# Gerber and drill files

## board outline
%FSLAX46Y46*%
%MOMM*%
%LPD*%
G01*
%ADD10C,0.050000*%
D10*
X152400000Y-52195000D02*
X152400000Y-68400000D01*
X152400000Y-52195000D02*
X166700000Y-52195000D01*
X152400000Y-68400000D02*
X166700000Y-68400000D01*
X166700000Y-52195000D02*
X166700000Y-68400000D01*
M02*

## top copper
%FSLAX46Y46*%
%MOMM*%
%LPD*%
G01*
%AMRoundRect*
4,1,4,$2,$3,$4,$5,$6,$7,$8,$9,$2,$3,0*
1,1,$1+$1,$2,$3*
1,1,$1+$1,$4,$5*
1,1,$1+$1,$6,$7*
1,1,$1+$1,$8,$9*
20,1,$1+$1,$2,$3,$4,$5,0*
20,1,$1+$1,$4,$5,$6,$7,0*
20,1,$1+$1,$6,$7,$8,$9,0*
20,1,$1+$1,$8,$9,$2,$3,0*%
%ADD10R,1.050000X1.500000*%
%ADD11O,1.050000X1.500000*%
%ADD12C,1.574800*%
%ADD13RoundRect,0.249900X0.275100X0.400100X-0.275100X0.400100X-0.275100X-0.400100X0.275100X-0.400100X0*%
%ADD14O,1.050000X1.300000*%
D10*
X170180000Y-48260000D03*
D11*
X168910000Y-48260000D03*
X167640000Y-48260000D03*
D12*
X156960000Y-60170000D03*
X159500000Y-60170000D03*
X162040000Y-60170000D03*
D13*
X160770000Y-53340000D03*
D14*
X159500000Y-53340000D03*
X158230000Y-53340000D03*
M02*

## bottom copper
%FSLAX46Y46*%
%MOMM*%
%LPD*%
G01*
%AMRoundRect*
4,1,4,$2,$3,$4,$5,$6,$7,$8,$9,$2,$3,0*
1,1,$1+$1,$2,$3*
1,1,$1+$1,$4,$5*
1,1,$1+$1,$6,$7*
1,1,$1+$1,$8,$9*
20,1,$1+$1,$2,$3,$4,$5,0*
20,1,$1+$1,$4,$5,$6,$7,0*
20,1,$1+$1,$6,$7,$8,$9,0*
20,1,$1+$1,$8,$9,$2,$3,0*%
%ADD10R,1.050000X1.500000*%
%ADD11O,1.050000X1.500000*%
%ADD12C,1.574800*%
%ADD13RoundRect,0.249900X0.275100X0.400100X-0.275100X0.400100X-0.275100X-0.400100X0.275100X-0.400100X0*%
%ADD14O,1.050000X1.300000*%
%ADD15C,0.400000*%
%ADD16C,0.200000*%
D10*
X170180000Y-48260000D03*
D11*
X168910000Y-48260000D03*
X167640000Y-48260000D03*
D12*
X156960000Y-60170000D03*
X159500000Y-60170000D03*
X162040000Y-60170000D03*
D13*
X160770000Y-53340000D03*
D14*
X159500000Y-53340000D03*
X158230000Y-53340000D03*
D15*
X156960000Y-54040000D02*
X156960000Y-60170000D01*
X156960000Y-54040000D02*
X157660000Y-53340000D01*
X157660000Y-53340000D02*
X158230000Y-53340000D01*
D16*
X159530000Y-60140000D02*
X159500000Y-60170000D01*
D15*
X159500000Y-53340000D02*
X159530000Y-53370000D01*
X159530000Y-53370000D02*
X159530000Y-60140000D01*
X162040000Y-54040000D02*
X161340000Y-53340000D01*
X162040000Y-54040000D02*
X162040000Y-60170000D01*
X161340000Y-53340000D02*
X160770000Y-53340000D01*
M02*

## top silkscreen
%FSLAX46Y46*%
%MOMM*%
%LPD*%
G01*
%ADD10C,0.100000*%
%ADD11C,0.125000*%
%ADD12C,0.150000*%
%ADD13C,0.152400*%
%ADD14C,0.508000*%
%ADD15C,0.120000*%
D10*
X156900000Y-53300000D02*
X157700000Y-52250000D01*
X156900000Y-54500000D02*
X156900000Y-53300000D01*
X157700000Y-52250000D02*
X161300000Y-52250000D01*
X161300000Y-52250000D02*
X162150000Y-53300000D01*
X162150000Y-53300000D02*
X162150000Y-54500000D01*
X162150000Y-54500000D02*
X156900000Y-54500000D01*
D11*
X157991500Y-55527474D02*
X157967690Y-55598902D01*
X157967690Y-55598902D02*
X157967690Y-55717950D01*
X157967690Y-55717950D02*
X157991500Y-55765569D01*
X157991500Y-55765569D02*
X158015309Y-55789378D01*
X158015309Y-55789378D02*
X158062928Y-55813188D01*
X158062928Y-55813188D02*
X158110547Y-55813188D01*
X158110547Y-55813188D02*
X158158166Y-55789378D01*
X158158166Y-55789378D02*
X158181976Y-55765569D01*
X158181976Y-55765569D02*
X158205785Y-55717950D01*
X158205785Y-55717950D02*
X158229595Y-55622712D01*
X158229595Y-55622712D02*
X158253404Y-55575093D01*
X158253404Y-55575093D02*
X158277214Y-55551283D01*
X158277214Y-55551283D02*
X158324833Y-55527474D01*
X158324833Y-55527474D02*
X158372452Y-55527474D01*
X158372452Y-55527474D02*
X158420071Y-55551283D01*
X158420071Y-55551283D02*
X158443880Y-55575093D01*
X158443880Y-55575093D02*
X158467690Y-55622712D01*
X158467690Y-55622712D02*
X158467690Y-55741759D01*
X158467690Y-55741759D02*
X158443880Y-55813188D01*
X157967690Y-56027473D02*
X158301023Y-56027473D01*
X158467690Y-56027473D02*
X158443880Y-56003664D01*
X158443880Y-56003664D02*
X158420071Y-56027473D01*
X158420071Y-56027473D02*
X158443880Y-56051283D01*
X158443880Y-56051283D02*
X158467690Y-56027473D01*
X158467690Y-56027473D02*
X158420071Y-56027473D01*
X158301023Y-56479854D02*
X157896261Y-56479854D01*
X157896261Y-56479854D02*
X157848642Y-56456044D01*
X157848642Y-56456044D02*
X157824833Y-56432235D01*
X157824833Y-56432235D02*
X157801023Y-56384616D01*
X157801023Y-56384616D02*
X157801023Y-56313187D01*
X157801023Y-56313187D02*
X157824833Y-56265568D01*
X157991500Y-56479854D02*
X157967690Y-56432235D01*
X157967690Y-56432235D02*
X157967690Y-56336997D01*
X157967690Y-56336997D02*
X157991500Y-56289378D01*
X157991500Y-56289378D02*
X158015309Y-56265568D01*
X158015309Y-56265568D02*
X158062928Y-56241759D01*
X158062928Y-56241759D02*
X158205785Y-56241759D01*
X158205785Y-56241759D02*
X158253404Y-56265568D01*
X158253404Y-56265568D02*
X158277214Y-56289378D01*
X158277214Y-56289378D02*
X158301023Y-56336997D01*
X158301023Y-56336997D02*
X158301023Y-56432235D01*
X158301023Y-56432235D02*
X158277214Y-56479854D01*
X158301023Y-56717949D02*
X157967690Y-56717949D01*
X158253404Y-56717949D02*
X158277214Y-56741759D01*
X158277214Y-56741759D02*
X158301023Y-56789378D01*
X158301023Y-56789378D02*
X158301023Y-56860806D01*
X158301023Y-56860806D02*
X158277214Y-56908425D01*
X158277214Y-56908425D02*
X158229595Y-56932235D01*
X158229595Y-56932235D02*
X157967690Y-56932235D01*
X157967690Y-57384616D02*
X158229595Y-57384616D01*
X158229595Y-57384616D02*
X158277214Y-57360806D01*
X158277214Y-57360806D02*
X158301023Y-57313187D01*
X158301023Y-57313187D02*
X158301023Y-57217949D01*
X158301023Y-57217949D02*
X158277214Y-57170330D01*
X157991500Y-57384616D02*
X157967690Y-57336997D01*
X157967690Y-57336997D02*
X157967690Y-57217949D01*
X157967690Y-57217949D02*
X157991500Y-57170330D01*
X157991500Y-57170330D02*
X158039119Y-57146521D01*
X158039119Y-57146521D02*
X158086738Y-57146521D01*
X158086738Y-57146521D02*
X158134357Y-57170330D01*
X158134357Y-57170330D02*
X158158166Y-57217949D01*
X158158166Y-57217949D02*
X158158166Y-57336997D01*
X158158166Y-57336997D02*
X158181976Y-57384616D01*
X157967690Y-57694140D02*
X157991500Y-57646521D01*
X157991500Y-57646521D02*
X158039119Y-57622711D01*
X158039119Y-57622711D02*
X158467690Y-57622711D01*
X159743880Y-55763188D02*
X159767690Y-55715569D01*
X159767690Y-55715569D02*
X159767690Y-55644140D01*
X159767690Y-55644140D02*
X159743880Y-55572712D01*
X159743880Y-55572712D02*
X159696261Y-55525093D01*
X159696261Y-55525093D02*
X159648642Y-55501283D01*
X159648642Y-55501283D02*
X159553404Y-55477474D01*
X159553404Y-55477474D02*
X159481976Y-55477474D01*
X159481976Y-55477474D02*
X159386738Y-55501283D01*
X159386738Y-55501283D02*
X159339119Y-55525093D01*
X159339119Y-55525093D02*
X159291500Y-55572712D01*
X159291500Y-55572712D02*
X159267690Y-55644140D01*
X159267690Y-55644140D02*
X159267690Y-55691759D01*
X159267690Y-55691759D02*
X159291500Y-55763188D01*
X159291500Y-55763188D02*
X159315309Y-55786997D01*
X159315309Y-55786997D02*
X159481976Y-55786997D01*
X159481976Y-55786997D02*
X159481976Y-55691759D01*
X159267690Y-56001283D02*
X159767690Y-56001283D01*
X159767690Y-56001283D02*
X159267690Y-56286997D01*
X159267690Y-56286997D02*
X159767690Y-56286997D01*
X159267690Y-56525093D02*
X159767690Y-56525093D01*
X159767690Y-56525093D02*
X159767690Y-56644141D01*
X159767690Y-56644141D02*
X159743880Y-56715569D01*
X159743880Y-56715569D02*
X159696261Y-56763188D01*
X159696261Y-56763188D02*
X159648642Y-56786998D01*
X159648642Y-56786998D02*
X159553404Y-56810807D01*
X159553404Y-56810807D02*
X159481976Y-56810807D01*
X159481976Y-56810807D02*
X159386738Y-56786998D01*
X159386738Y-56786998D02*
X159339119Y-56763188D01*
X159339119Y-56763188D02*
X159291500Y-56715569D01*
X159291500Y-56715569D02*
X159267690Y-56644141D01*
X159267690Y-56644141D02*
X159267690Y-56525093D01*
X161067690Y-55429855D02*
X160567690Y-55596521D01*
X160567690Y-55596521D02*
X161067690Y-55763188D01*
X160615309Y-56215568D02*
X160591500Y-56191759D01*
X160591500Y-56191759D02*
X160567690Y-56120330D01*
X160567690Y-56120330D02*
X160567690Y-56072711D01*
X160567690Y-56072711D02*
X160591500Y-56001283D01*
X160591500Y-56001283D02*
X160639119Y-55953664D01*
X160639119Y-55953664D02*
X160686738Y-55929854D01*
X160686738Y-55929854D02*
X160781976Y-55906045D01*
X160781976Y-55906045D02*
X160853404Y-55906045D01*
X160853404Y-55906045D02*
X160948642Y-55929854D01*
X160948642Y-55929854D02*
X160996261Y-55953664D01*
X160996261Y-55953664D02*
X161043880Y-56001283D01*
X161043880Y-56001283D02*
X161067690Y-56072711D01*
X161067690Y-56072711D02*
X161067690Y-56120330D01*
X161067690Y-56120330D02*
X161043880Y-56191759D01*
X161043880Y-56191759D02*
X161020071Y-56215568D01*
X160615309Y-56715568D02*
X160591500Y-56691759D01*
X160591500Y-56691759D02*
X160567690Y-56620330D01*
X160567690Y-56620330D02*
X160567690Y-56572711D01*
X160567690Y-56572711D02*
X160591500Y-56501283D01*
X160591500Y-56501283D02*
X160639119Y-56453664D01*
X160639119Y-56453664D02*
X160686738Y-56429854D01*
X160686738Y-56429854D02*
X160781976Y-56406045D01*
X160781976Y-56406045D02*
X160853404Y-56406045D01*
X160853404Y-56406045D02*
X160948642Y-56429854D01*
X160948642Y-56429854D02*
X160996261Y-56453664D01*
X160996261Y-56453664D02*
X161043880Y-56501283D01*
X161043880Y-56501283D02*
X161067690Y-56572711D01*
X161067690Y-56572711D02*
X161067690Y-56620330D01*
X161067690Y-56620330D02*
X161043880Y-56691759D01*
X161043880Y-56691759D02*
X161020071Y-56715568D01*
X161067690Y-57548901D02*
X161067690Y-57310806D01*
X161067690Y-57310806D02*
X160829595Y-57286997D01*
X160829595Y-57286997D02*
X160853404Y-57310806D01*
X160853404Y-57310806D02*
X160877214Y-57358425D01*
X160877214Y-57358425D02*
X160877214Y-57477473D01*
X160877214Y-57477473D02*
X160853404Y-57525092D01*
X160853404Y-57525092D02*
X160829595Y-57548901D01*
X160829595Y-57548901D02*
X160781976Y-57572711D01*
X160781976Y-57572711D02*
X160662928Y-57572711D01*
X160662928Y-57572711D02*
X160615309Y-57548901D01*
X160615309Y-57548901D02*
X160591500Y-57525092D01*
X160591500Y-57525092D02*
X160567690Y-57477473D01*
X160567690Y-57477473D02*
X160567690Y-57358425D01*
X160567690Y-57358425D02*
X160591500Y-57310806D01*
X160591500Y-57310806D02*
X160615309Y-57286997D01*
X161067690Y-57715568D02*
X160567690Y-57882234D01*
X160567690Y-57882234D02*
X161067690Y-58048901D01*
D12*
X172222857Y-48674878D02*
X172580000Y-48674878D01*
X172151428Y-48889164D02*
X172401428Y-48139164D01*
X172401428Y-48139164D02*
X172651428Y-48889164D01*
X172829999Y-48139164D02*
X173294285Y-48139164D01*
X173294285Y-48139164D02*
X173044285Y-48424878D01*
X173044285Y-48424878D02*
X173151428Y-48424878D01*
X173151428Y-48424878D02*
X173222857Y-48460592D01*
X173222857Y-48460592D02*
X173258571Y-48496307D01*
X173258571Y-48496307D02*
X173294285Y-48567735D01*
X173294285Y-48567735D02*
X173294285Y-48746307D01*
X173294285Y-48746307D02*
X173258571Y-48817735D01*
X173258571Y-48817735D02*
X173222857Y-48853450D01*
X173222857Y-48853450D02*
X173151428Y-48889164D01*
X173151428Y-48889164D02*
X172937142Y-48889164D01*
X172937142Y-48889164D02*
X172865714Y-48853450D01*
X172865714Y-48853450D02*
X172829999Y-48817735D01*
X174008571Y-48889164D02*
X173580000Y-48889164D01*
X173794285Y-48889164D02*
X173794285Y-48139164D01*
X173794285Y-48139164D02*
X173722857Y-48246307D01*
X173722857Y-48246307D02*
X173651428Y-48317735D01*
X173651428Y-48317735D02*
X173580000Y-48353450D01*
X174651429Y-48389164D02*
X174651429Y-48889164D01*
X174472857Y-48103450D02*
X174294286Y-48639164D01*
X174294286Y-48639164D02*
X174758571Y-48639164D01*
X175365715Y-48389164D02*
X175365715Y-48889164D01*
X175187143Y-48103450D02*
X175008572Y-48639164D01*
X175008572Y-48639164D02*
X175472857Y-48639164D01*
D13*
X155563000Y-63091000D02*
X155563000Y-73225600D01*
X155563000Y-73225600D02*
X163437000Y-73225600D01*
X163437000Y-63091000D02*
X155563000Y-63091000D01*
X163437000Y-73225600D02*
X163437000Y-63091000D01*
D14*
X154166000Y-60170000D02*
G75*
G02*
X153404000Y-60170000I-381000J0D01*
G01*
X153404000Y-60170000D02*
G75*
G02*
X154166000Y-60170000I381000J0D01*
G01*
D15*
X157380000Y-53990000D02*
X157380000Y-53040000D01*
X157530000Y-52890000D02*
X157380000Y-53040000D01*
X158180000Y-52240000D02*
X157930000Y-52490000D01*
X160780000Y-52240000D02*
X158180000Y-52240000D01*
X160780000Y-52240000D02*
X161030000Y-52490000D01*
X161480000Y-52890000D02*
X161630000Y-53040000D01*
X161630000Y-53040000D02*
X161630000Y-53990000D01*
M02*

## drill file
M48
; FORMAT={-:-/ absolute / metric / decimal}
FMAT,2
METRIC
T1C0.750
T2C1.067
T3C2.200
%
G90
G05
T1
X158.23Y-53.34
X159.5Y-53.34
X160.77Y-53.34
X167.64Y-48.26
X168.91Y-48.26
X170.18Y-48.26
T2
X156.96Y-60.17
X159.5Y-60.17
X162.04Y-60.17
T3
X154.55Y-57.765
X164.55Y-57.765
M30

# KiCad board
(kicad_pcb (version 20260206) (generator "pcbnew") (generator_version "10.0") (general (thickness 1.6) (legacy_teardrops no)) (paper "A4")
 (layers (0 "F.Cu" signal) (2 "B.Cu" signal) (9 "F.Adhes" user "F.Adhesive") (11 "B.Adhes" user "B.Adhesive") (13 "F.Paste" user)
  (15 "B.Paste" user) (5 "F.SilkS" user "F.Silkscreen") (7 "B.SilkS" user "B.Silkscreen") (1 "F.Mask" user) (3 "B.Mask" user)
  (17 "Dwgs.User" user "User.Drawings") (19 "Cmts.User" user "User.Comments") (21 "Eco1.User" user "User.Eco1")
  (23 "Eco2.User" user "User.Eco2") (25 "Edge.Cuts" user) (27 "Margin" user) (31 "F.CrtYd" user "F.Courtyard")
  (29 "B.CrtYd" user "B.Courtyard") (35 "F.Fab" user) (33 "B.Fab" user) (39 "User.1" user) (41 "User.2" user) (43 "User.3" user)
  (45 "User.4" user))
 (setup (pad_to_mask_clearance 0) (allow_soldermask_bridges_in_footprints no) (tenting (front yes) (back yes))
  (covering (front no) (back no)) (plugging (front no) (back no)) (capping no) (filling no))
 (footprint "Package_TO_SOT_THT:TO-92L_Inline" (layer "F.Cu") (at 170.18 48.26 180)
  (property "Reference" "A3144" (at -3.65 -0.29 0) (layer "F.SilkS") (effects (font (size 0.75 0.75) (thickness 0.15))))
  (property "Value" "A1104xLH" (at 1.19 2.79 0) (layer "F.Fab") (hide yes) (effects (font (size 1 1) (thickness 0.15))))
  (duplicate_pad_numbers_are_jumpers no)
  (pad "1" thru_hole rect (at 0 0 180) (size 1.05 1.5) (drill 0.75) (layers "*.Cu" "*.Mask") (remove_unused_layers no)
   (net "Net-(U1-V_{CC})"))
  (pad "2" thru_hole oval (at 1.27 0 180) (size 1.05 1.5) (drill 0.75) (layers "*.Cu" "*.Mask") (remove_unused_layers no)
   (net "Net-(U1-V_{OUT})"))
  (pad "3" thru_hole oval (at 2.54 0 180) (size 1.05 1.5) (drill 0.75) (layers "*.Cu" "*.Mask") (remove_unused_layers no)
   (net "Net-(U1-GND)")))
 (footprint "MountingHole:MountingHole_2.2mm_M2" (layer "F.Cu") (at 164.55 57.765)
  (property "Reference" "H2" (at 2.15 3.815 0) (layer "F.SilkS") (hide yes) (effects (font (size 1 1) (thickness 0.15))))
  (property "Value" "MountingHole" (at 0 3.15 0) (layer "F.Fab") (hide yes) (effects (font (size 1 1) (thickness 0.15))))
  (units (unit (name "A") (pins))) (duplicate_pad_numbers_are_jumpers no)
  (pad "" np_thru_hole circle (at 0 0) (size 2.2 2.2) (drill 2.2) (layers "*.Cu" "*.Mask")))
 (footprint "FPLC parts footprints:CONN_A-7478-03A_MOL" (layer "F.Cu") (at 156.96 60.17)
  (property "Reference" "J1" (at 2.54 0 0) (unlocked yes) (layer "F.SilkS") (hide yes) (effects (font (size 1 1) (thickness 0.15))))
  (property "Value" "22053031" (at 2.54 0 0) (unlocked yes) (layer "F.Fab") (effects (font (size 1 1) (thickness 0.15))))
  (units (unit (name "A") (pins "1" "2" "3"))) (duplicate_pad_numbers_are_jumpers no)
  (fp_line (start -1.397 2.921) (end -1.397 13.0556) (stroke (width 0.1524) (type solid)) (layer "F.SilkS"))
  (fp_line (start -1.397 13.0556) (end 6.477 13.0556) (stroke (width 0.1524) (type solid)) (layer "F.SilkS"))
  (fp_line (start 6.477 2.921) (end -1.397 2.921) (stroke (width 0.1524) (type solid)) (layer "F.SilkS"))
  (fp_line (start 6.477 13.0556) (end 6.477 2.921) (stroke (width 0.1524) (type solid)) (layer "F.SilkS"))
  (fp_circle (center -3.175 0) (end -2.794 0) (stroke (width 0.508) (type solid)) (fill no) (layer "F.SilkS"))
  (pad "1" thru_hole circle (at 0 0) (size 1.5748 1.5748) (drill 1.0668) (layers "*.Cu" "*.Mask") (remove_unused_layers no) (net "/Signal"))
  (pad "2" thru_hole circle (at 2.54 0) (size 1.5748 1.5748) (drill 1.0668) (layers "*.Cu" "*.Mask") (remove_unused_layers no) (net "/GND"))
  (pad "3" thru_hole circle (at 5.08 0) (size 1.5748 1.5748) (drill 1.0668) (layers "*.Cu" "*.Mask") (remove_unused_layers no)
   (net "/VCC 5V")))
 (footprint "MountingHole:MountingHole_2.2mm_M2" (layer "F.Cu") (at 154.55 57.765)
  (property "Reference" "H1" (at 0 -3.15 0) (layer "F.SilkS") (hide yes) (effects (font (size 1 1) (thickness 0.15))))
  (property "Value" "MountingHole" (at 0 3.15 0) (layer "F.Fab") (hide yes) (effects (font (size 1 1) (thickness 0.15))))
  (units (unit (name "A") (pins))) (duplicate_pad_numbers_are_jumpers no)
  (pad "" np_thru_hole circle (at 0 0) (size 2.2 2.2) (drill 2.2) (layers "*.Cu" "*.Mask")))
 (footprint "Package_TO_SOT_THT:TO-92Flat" (layer "F.Cu") (at 160.77 53.34 180)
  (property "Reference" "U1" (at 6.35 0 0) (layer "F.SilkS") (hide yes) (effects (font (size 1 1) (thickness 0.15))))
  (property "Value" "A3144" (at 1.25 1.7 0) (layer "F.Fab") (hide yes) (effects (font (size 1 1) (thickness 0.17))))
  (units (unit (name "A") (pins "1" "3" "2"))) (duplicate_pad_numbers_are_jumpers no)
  (fp_line (start 3.39 -0.65) (end 3.39 0.3) (stroke (width 0.12) (type solid)) (layer "F.SilkS"))
  (fp_line (start 3.24 0.45) (end 3.39 0.3) (stroke (width 0.12) (type solid)) (layer "F.SilkS"))
  (fp_line (start 2.59 1.1) (end 2.84 0.85) (stroke (width 0.12) (type solid)) (layer "F.SilkS"))
  (fp_line (start -0.01 1.1) (end 2.59 1.1) (stroke (width 0.12) (type solid)) (layer "F.SilkS"))
  (fp_line (start -0.01 1.1) (end -0.26 0.85) (stroke (width 0.12) (type solid)) (layer "F.SilkS"))
  (fp_line (start -0.71 0.45) (end -0.86 0.3) (stroke (width 0.12) (type solid)) (layer "F.SilkS"))
  (fp_line (start -0.86 0.3) (end -0.86 -0.65) (stroke (width 0.12) (type solid)) (layer "F.SilkS"))
  (pad "1" thru_hole roundrect (at 0 0 180) (size 1.05 1.3) (drill 0.75) (layers "*.Cu" "*.Mask") (remove_unused_layers no)
   (roundrect_rratio 0.238) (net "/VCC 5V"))
  (pad "2" thru_hole oval (at 1.27 0 180) (size 1.05 1.3) (drill 0.75) (layers "*.Cu" "*.Mask") (remove_unused_layers no) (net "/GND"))
  (pad "3" thru_hole oval (at 2.54 0 180) (size 1.05 1.3) (drill 0.75) (layers "*.Cu" "*.Mask") (remove_unused_layers no) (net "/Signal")))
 (gr_line (start 156.9 53.3) (end 157.7 52.25) (stroke (width 0.1) (type default)) (layer "F.SilkS"))
 (gr_line (start 156.9 54.5) (end 156.9 53.3) (stroke (width 0.1) (type default)) (layer "F.SilkS"))
 (gr_line (start 157.7 52.25) (end 161.3 52.25) (stroke (width 0.1) (type default)) (layer "F.SilkS"))
 (gr_line (start 161.3 52.25) (end 162.15 53.3) (stroke (width 0.1) (type default)) (layer "F.SilkS"))
 (gr_line (start 162.15 53.3) (end 162.15 54.5) (stroke (width 0.1) (type default)) (layer "F.SilkS"))
 (gr_line (start 162.15 54.5) (end 156.9 54.5) (stroke (width 0.1) (type default)) (layer "F.SilkS"))
 (gr_line (start 152.4 52.195) (end 152.4 68.4) (stroke (width 0.05) (type solid)) (layer "Edge.Cuts"))
 (gr_line (start 152.4 52.195) (end 166.7 52.195) (stroke (width 0.05) (type solid)) (layer "Edge.Cuts"))
 (gr_line (start 152.4 68.4) (end 166.7 68.4) (stroke (width 0.05) (type solid)) (layer "Edge.Cuts"))
 (gr_line (start 166.7 52.195) (end 166.7 68.4) (stroke (width 0.05) (type solid)) (layer "Edge.Cuts"))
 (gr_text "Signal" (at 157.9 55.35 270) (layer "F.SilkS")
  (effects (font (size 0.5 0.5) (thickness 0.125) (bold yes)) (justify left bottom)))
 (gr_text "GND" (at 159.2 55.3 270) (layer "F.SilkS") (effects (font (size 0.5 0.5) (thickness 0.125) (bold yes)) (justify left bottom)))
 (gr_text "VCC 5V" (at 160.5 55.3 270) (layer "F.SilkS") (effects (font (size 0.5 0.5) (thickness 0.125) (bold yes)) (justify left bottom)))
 (segment (start 156.96 54.04) (end 156.96 60.17) (width 0.4) (layer "B.Cu") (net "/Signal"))
 (segment (start 156.96 54.04) (end 157.66 53.34) (width 0.4) (layer "B.Cu") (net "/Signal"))
 (segment (start 157.66 53.34) (end 158.23 53.34) (width 0.4) (layer "B.Cu") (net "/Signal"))
 (segment (start 159.53 60.14) (end 159.5 60.17) (width 0.2) (layer "B.Cu") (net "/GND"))
 (segment (start 159.5 53.34) (end 159.53 53.37) (width 0.4) (layer "B.Cu") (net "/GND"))
 (segment (start 159.53 53.37) (end 159.53 60.14) (width 0.4) (layer "B.Cu") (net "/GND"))
 (segment (start 162.04 54.04) (end 161.34 53.34) (width 0.4) (layer "B.Cu") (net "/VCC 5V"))
 (segment (start 162.04 54.04) (end 162.04 60.17) (width 0.4) (layer "B.Cu") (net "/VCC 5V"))
 (segment (start 161.34 53.34) (end 160.77 53.34) (width 0.4) (layer "B.Cu") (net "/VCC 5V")))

